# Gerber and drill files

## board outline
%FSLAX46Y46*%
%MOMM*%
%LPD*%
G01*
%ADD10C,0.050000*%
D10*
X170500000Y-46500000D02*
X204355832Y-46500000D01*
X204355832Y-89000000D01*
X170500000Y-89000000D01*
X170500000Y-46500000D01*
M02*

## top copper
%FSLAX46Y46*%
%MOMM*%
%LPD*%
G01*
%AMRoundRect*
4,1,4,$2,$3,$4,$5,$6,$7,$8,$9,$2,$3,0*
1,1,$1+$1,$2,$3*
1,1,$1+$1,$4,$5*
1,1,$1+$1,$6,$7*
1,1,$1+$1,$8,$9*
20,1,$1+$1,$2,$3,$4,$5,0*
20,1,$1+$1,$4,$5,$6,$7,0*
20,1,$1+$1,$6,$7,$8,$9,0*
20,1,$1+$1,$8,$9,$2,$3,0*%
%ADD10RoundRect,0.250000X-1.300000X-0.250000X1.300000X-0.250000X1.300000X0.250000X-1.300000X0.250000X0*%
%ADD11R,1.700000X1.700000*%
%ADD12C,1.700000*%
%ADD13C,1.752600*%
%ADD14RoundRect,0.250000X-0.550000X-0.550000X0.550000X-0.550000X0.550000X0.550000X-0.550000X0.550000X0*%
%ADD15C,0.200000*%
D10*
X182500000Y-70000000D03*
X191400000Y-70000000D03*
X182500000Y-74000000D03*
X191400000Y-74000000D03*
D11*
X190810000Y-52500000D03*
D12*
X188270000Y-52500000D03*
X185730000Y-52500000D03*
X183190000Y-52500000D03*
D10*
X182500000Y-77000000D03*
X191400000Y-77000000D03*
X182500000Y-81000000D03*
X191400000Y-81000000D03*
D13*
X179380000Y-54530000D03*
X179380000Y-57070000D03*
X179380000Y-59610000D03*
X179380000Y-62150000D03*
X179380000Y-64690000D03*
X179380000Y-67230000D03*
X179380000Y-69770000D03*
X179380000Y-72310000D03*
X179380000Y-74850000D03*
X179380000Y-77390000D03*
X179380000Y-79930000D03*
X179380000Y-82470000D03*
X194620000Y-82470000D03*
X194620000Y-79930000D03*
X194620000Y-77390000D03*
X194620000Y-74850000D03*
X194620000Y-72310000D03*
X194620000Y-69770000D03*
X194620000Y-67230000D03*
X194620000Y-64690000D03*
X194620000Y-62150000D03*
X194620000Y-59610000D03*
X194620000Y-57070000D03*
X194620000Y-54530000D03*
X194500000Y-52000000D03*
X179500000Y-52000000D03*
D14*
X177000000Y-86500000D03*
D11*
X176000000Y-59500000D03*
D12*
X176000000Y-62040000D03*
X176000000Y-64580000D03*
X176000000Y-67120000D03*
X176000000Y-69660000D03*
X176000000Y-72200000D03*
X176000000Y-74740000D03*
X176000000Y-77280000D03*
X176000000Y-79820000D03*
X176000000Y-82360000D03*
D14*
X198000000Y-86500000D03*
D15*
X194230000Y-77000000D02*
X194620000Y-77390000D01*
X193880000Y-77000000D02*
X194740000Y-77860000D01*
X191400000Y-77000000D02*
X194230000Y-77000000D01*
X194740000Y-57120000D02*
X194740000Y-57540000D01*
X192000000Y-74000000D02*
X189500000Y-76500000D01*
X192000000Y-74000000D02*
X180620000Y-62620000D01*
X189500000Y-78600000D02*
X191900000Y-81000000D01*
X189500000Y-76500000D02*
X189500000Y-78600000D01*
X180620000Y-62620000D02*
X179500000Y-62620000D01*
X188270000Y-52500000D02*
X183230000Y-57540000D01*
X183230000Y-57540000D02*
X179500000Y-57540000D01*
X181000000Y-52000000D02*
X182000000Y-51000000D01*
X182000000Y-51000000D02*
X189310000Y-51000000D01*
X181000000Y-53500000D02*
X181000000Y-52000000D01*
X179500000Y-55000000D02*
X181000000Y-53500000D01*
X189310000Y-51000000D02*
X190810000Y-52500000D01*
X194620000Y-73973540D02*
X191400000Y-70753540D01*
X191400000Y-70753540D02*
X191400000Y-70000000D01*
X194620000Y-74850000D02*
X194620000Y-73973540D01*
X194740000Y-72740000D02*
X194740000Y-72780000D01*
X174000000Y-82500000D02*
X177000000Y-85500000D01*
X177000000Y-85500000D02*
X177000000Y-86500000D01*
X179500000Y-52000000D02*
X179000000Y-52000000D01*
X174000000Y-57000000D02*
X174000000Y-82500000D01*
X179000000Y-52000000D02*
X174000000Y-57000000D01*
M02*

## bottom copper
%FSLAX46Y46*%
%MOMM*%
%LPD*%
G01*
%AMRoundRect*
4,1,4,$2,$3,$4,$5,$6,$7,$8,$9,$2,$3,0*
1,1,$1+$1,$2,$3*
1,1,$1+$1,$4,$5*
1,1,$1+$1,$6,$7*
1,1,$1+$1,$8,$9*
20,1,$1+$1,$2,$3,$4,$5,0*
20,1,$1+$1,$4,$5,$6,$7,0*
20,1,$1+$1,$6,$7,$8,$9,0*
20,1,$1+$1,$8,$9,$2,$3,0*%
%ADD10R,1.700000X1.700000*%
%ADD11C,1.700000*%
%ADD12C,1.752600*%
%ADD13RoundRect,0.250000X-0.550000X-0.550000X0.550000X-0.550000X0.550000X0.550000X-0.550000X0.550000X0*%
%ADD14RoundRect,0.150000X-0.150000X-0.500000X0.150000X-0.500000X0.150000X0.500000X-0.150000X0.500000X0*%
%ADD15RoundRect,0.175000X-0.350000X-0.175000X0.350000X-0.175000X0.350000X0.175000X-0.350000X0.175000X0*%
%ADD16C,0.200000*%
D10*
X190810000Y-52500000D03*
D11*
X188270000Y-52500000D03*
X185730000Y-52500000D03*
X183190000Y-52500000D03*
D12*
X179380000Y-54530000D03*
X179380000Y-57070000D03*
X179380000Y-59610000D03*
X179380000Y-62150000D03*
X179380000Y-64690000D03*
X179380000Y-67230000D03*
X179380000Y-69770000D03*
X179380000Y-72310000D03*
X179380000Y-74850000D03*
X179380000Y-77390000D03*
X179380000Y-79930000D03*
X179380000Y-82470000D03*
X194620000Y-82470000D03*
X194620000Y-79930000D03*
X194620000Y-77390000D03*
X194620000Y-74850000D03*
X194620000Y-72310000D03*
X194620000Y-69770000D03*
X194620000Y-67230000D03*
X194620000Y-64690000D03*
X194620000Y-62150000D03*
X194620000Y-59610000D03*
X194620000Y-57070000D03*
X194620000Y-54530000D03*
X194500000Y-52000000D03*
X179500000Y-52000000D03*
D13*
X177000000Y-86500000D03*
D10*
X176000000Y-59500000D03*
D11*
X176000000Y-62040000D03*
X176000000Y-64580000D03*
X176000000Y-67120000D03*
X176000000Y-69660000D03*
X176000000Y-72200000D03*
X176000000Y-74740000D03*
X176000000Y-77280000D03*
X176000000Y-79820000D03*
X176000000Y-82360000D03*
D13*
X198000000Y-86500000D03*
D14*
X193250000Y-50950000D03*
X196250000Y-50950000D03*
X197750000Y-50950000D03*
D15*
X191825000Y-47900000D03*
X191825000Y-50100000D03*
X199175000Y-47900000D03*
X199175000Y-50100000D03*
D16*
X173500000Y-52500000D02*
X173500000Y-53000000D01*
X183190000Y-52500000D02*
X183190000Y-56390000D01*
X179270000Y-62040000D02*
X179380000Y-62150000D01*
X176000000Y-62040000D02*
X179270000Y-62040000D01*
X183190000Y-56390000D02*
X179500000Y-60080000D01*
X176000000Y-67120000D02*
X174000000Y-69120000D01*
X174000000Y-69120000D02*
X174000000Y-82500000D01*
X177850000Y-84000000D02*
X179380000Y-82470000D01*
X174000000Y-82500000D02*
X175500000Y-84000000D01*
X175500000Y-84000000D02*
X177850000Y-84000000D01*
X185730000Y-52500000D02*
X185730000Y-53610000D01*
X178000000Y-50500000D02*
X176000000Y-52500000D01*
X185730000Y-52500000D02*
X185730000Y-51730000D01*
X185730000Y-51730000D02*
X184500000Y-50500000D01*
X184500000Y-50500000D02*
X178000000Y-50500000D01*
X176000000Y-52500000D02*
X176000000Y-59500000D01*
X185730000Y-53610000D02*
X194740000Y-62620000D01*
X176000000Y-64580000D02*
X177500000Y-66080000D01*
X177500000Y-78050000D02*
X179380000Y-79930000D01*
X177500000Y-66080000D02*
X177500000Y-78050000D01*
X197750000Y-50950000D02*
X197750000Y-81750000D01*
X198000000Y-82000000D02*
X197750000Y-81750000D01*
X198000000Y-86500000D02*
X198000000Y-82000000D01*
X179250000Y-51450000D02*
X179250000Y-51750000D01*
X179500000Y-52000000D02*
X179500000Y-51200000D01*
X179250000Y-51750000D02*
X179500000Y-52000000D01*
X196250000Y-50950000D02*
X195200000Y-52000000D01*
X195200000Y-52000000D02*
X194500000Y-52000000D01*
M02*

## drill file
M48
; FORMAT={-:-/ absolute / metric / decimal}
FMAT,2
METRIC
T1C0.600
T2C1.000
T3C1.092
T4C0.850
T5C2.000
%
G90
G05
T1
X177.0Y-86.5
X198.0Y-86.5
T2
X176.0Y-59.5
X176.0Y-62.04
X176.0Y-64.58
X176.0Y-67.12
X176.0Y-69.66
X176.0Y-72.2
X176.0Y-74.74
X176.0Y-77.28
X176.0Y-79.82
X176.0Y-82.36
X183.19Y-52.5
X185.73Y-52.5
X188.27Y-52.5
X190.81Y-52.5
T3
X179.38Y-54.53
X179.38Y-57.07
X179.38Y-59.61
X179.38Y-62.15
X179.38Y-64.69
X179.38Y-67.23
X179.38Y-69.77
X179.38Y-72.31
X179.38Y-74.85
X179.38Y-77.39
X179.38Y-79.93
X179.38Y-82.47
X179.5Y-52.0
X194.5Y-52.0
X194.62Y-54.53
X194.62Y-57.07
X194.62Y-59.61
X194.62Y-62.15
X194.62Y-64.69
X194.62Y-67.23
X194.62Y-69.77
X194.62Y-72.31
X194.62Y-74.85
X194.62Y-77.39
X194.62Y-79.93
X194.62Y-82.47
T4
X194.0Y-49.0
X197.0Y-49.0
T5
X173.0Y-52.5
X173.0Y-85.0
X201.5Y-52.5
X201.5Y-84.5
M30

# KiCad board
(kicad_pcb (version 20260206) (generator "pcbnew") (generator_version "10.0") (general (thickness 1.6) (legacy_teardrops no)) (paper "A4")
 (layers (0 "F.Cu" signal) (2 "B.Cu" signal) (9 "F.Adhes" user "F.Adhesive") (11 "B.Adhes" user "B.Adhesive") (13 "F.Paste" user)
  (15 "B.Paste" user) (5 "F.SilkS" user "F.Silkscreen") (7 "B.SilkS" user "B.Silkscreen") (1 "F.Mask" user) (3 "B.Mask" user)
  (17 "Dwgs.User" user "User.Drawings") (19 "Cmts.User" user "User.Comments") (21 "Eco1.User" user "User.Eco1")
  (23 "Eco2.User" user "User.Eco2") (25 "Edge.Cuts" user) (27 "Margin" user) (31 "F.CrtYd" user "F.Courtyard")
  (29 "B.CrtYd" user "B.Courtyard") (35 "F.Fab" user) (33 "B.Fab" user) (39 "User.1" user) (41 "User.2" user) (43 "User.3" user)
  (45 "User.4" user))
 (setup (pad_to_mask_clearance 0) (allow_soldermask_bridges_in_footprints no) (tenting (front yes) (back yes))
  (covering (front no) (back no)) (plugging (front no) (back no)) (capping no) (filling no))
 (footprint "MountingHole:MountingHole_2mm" (layer "F.Cu") (at 201.5 52.5)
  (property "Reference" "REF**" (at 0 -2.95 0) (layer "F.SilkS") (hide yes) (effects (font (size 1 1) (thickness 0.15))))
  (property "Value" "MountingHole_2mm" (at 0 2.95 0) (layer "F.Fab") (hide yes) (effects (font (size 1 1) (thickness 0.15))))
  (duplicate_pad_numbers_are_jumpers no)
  (pad "" np_thru_hole circle (at 0 0) (size 2 2) (drill 2) (layers "*.Cu" "*.Mask")))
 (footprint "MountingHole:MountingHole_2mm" (layer "F.Cu") (at 201.5 84.5)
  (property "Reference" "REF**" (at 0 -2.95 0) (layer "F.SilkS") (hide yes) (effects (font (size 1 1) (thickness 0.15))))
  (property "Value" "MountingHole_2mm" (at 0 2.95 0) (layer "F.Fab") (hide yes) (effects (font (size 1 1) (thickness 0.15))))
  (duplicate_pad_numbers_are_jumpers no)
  (pad "" np_thru_hole circle (at 0 0) (size 2 2) (drill 2) (layers "*.Cu" "*.Mask")))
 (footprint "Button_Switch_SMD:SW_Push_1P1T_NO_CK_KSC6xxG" (layer "F.Cu") (at 186.95 72)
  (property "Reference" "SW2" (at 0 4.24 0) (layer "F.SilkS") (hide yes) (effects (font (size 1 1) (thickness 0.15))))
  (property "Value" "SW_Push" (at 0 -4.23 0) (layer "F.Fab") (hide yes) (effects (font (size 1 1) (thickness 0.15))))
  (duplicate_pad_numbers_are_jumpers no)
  (pad "1" smd roundrect (at -4.45 -2) (size 3.1 1) (layers "F.Cu" "F.Mask" "F.Paste") (roundrect_rratio 0.25) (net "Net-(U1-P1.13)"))
  (pad "1" smd roundrect (at 4.45 -2) (size 3.1 1) (layers "F.Cu" "F.Mask" "F.Paste") (roundrect_rratio 0.25) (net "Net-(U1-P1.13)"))
  (pad "2" smd roundrect (at -4.45 2) (size 3.1 1) (layers "F.Cu" "F.Mask" "F.Paste") (roundrect_rratio 0.25) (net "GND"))
  (pad "2" smd roundrect (at 4.45 2) (size 3.1 1) (layers "F.Cu" "F.Mask" "F.Paste") (roundrect_rratio 0.25) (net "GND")))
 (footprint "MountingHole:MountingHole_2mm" (layer "F.Cu") (at 173 52.5)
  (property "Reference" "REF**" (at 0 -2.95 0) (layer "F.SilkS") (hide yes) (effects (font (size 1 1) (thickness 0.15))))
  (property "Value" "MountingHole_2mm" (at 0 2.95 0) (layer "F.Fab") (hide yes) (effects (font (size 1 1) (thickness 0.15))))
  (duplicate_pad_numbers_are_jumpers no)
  (pad "" np_thru_hole circle (at 0 0) (size 2 2) (drill 2) (layers "*.Cu" "*.Mask")))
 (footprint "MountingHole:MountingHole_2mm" (layer "F.Cu") (at 173 85)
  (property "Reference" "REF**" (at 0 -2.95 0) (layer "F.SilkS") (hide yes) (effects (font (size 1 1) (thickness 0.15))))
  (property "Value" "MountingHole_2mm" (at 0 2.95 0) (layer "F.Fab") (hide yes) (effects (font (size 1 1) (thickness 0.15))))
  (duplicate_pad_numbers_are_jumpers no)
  (pad "" np_thru_hole circle (at 0 0) (size 2 2) (drill 2) (layers "*.Cu" "*.Mask")))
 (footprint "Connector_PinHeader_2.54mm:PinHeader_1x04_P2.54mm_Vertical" (layer "F.Cu") (at 190.81 52.5 -90)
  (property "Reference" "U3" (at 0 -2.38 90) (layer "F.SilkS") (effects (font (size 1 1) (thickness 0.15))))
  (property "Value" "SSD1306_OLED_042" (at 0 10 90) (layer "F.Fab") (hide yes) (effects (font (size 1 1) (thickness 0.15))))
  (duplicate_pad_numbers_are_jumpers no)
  (pad "1" thru_hole rect (at 0 0 270) (size 1.7 1.7) (drill 1) (layers "*.Cu" "*.Mask") (remove_unused_layers no)
   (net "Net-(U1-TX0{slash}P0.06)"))
  (pad "2" thru_hole circle (at 0 2.54 270) (size 1.7 1.7) (drill 1) (layers "*.Cu" "*.Mask") (remove_unused_layers no)
   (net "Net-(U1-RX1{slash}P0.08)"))
  (pad "3" thru_hole circle (at 0 5.08 270) (size 1.7 1.7) (drill 1) (layers "*.Cu" "*.Mask") (remove_unused_layers no) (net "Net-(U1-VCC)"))
  (pad "4" thru_hole circle (at 0 7.62 270) (size 1.7 1.7) (drill 1) (layers "*.Cu" "*.Mask") (remove_unused_layers no) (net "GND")))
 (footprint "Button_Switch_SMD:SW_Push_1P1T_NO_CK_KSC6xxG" (layer "F.Cu") (at 186.95 79)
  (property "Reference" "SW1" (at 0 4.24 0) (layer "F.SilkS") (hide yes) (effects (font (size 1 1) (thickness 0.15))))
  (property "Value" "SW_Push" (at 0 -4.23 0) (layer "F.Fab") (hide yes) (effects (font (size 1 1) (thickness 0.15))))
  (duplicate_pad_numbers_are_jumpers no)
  (pad "1" smd roundrect (at -4.45 -2) (size 3.1 1) (layers "F.Cu" "F.Mask" "F.Paste") (roundrect_rratio 0.25) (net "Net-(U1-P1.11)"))
  (pad "1" smd roundrect (at 4.45 -2) (size 3.1 1) (layers "F.Cu" "F.Mask" "F.Paste") (roundrect_rratio 0.25) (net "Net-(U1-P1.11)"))
  (pad "2" smd roundrect (at -4.45 2) (size 3.1 1) (layers "F.Cu" "F.Mask" "F.Paste") (roundrect_rratio 0.25) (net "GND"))
  (pad "2" smd roundrect (at 4.45 2) (size 3.1 1) (layers "F.Cu" "F.Mask" "F.Paste") (roundrect_rratio 0.25) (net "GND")))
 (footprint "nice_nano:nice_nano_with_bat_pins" (layer "F.Cu") (at 187 68.5 -90)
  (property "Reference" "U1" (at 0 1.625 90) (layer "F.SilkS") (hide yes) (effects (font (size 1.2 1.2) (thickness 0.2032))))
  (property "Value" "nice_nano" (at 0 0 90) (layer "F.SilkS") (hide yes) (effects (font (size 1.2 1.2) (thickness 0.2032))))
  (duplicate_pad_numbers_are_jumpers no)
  (pad "1" thru_hole circle (at -13.97 7.62 270) (size 1.7526 1.7526) (drill 1.0922) (layers "*.Cu" "*.SilkS" "*.Mask")
   (remove_unused_layers no) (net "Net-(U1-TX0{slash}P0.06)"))
  (pad "2" thru_hole circle (at -11.43 7.62 270) (size 1.7526 1.7526) (drill 1.0922) (layers "*.Cu" "*.SilkS" "*.Mask")
   (remove_unused_layers no) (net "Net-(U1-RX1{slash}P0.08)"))
  (pad "3" thru_hole circle (at -8.89 7.62 270) (size 1.7526 1.7526) (drill 1.0922) (layers "*.Cu" "*.SilkS" "*.Mask")
   (remove_unused_layers no) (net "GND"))
  (pad "4" thru_hole circle (at -6.35 7.62 270) (size 1.7526 1.7526) (drill 1.0922) (layers "*.Cu" "*.SilkS" "*.Mask")
   (remove_unused_layers no) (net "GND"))
  (pad "5" thru_hole circle (at -3.81 7.62 270) (size 1.7526 1.7526) (drill 1.0922) (layers "*.Cu" "*.SilkS" "*.Mask")
   (remove_unused_layers no) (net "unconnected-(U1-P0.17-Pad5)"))
  (pad "6" thru_hole circle (at -1.27 7.62 270) (size 1.7526 1.7526) (drill 1.0922) (layers "*.Cu" "*.SilkS" "*.Mask")
   (remove_unused_layers no) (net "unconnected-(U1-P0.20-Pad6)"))
  (pad "7" thru_hole circle (at 1.27 7.62 270) (size 1.7526 1.7526) (drill 1.0922) (layers "*.Cu" "*.SilkS" "*.Mask")
   (remove_unused_layers no) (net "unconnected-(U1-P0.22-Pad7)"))
  (pad "8" thru_hole circle (at 3.81 7.62 270) (size 1.7526 1.7526) (drill 1.0922) (layers "*.Cu" "*.SilkS" "*.Mask")
   (remove_unused_layers no) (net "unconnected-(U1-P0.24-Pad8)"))
  (pad "9" thru_hole circle (at 6.35 7.62 270) (size 1.7526 1.7526) (drill 1.0922) (layers "*.Cu" "*.SilkS" "*.Mask")
   (remove_unused_layers no) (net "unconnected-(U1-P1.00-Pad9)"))
  (pad "10" thru_hole circle (at 8.89 7.62 270) (size 1.7526 1.7526) (drill 1.0922) (layers "*.Cu" "*.SilkS" "*.Mask")
   (remove_unused_layers no) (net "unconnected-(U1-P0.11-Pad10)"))
  (pad "11" thru_hole circle (at 11.43 7.62 270) (size 1.7526 1.7526) (drill 1.0922) (layers "*.Cu" "*.SilkS" "*.Mask")
   (remove_unused_layers no) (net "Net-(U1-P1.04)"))
  (pad "12" thru_hole circle (at 13.97 7.62 270) (size 1.7526 1.7526) (drill 1.0922) (layers "*.Cu" "*.SilkS" "*.Mask")
   (remove_unused_layers no) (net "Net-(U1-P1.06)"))
  (pad "13" thru_hole circle (at 13.97 -7.62 270) (size 1.7526 1.7526) (drill 1.0922) (layers "*.Cu" "*.SilkS" "*.Mask")
   (remove_unused_layers no) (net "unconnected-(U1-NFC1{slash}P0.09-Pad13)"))
  (pad "14" thru_hole circle (at 11.43 -7.62 270) (size 1.7526 1.7526) (drill 1.0922) (layers "*.Cu" "*.SilkS" "*.Mask")
   (remove_unused_layers no) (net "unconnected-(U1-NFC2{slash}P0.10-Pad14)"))
  (pad "15" thru_hole circle (at 8.89 -7.62 270) (size 1.7526 1.7526) (drill 1.0922) (layers "*.Cu" "*.SilkS" "*.Mask")
   (remove_unused_layers no) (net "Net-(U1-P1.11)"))
  (pad "16" thru_hole circle (at 6.35 -7.62 270) (size 1.7526 1.7526) (drill 1.0922) (layers "*.Cu" "*.SilkS" "*.Mask")
   (remove_unused_layers no) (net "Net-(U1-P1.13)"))
  (pad "17" thru_hole circle (at 3.81 -7.62 270) (size 1.7526 1.7526) (drill 1.0922) (layers "*.Cu" "*.SilkS" "*.Mask")
   (remove_unused_layers no) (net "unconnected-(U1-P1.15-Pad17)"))
  (pad "18" thru_hole circle (at 1.27 -7.62 270) (size 1.7526 1.7526) (drill 1.0922) (layers "*.Cu" "*.SilkS" "*.Mask")
   (remove_unused_layers no) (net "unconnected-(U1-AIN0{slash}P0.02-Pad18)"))
  (pad "19" thru_hole circle (at -1.27 -7.62 270) (size 1.7526 1.7526) (drill 1.0922) (layers "*.Cu" "*.SilkS" "*.Mask")
   (remove_unused_layers no) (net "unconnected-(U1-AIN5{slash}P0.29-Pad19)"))
  (pad "20" thru_hole circle (at -3.81 -7.62 270) (size 1.7526 1.7526) (drill 1.0922) (layers "*.Cu" "*.SilkS" "*.Mask")
   (remove_unused_layers no) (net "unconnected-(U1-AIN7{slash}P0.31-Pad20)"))
  (pad "21" thru_hole circle (at -6.35 -7.62 270) (size 1.7526 1.7526) (drill 1.0922) (layers "*.Cu" "*.SilkS" "*.Mask")
   (remove_unused_layers no) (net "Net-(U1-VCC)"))
  (pad "22" thru_hole circle (at -8.89 -7.62 270) (size 1.7526 1.7526) (drill 1.0922) (layers "*.Cu" "*.SilkS" "*.Mask")
   (remove_unused_layers no) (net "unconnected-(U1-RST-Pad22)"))
  (pad "23" thru_hole circle (at -11.43 -7.62 270) (size 1.7526 1.7526) (drill 1.0922) (layers "*.Cu" "*.SilkS" "*.Mask")
   (remove_unused_layers no) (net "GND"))
  (pad "24" thru_hole circle (at -13.97 -7.62 270) (size 1.7526 1.7526) (drill 1.0922) (layers "*.Cu" "*.SilkS" "*.Mask")
   (remove_unused_layers no) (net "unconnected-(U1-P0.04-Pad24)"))
  (pad "25" thru_hole circle (at -16.5 -7.5 270) (size 1.7526 1.7526) (drill 1.0922) (layers "*.Cu" "*.SilkS" "*.Mask")
   (remove_unused_layers no) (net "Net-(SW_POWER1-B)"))
  (pad "26" thru_hole circle (at -16.5 7.5 270) (size 1.7526 1.7526) (drill 1.0922) (layers "*.Cu" "*.SilkS" "*.Mask")
   (remove_unused_layers no) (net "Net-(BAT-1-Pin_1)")))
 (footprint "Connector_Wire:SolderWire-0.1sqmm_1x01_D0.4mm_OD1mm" (layer "B.Cu") (at 177 86.5)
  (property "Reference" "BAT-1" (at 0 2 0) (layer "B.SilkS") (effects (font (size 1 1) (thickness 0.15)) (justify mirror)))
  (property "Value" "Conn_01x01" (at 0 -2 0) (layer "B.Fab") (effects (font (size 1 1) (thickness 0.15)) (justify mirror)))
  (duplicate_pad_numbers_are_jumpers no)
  (pad "1" thru_hole roundrect (at 0 0) (size 1.6 1.6) (drill 0.6) (layers "*.Cu" "*.Mask") (remove_unused_layers no)
   (roundrect_rratio 0.15625) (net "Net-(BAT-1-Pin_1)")))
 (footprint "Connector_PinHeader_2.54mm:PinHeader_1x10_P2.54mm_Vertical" (layer "B.Cu") (at 176 59.5 180)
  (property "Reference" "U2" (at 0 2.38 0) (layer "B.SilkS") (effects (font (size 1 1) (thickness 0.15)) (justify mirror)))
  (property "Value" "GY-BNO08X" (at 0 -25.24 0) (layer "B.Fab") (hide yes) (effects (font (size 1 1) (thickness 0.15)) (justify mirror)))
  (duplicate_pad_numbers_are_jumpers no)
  (pad "1" thru_hole rect (at 0 0 180) (size 1.7 1.7) (drill 1) (layers "*.Cu" "*.Mask") (remove_unused_layers no) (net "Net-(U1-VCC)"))
  (pad "2" thru_hole circle (at 0 -2.54 180) (size 1.7 1.7) (drill 1) (layers "*.Cu" "*.Mask") (remove_unused_layers no) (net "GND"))
  (pad "3" thru_hole circle (at 0 -5.08 180) (size 1.7 1.7) (drill 1) (layers "*.Cu" "*.Mask") (remove_unused_layers no)
   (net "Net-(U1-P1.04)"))
  (pad "4" thru_hole circle (at 0 -7.62 180) (size 1.7 1.7) (drill 1) (layers "*.Cu" "*.Mask") (remove_unused_layers no)
   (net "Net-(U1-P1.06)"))
  (pad "5" thru_hole circle (at 0 -10.16 180) (size 1.7 1.7) (drill 1) (layers "*.Cu" "*.Mask") (remove_unused_layers no)
   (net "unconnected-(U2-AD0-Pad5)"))
  (pad "6" thru_hole circle (at 0 -12.7 180) (size 1.7 1.7) (drill 1) (layers "*.Cu" "*.Mask") (remove_unused_layers no)
   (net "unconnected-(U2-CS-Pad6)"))
  (pad "7" thru_hole circle (at 0 -15.24 180) (size 1.7 1.7) (drill 1) (layers "*.Cu" "*.Mask") (remove_unused_layers no)
   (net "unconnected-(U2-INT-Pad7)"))
  (pad "8" thru_hole circle (at 0 -17.78 180) (size 1.7 1.7) (drill 1) (layers "*.Cu" "*.Mask") (remove_unused_layers no)
   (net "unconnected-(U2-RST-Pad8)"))
  (pad "9" thru_hole circle (at 0 -20.32 180) (size 1.7 1.7) (drill 1) (layers "*.Cu" "*.Mask") (remove_unused_layers no)
   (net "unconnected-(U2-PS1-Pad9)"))
  (pad "10" thru_hole circle (at 0 -22.86 180) (size 1.7 1.7) (drill 1) (layers "*.Cu" "*.Mask") (remove_unused_layers no)
   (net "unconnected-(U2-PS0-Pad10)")))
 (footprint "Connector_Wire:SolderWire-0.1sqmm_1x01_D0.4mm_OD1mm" (layer "B.Cu") (at 198 86.5)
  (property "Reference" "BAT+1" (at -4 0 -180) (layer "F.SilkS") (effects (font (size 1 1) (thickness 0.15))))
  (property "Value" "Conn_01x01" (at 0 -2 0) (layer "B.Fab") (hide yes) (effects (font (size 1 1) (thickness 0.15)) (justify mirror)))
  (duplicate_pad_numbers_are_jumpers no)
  (pad "1" thru_hole roundrect (at 0 0) (size 1.6 1.6) (drill 0.6) (layers "*.Cu" "*.Mask") (remove_unused_layers no)
   (roundrect_rratio 0.15625) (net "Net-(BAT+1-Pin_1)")))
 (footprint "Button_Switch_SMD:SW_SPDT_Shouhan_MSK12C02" (layer "B.Cu") (at 195.5 49)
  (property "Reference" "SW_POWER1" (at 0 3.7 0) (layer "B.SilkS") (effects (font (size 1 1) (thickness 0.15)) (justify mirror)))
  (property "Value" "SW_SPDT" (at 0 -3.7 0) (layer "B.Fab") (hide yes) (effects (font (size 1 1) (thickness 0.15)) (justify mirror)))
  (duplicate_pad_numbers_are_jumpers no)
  (pad "" np_thru_hole circle (at -1.5 0) (size 0.85 0.85) (drill 0.85) (layers "*.Mask"))
  (pad "" np_thru_hole circle (at 1.5 0) (size 0.85 0.85) (drill 0.85) (layers "*.Mask"))
  (pad "1" smd roundrect (at -2.25 1.95) (size 0.6 1.3) (layers "B.Cu" "B.Mask" "B.Paste") (roundrect_rratio 0.25)
   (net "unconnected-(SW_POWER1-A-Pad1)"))
  (pad "2" smd roundrect (at 0.75 1.95) (size 0.6 1.3) (layers "B.Cu" "B.Mask" "B.Paste") (roundrect_rratio 0.25) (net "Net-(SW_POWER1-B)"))
  (pad "3" smd roundrect (at 2.25 1.95) (size 0.6 1.3) (layers "B.Cu" "B.Mask" "B.Paste") (roundrect_rratio 0.25) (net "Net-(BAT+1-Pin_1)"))
  (pad "SH" smd roundrect (at -3.675 -1.1) (size 1.05 0.7) (layers "B.Cu" "B.Mask" "B.Paste") (roundrect_rratio 0.25))
  (pad "SH" smd roundrect (at -3.675 1.1) (size 1.05 0.7) (layers "B.Cu" "B.Mask" "B.Paste") (roundrect_rratio 0.25))
  (pad "SH" smd roundrect (at 3.675 -1.1) (size 1.05 0.7) (layers "B.Cu" "B.Mask" "B.Paste") (roundrect_rratio 0.25))
  (pad "SH" smd roundrect (at 3.675 1.1) (size 1.05 0.7) (layers "B.Cu" "B.Mask" "B.Paste") (roundrect_rratio 0.25)))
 (gr_rect (start 170.5 46.5) (end 204.355832 89) (stroke (width 0.05) (type default)) (fill no) (layer "Edge.Cuts"))
 (segment (start 173.5 52.5) (end 173.5 53) (width 0.2) (layer "B.Cu") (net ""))
 (segment (start 194.23 77) (end 194.62 77.39) (width 0.2) (layer "F.Cu") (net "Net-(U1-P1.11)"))
 (segment (start 193.88 77) (end 194.74 77.86) (width 0.2) (layer "F.Cu") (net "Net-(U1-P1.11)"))
 (segment (start 191.4 77) (end 194.23 77) (width 0.2) (layer "F.Cu") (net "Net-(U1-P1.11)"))
 (segment (start 194.74 57.12) (end 194.74 57.54) (width 0.2) (layer "F.Cu") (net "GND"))
 (segment (start 192 74) (end 189.5 76.5) (width 0.2) (layer "F.Cu") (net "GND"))
 (segment (start 192 74) (end 180.62 62.62) (width 0.2) (layer "F.Cu") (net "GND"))
 (segment (start 189.5 78.6) (end 191.9 81) (width 0.2) (layer "F.Cu") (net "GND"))
 (segment (start 189.5 76.5) (end 189.5 78.6) (width 0.2) (layer "F.Cu") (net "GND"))
 (segment (start 180.62 62.62) (end 179.5 62.62) (width 0.2) (layer "F.Cu") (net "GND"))
 (segment (start 183.19 52.5) (end 183.19 56.39) (width 0.2) (layer "B.Cu") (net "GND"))
 (segment (start 179.27 62.04) (end 179.38 62.15) (width 0.2) (layer "B.Cu") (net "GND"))
 (segment (start 176 62.04) (end 179.27 62.04) (width 0.2) (layer "B.Cu") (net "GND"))
 (segment (start 183.19 56.39) (end 179.5 60.08) (width 0.2) (layer "B.Cu") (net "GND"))
 (segment (start 176 67.12) (end 174 69.12) (width 0.2) (layer "B.Cu") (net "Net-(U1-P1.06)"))
 (segment (start 174 69.12) (end 174 82.5) (width 0.2) (layer "B.Cu") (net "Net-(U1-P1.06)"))
 (segment (start 177.85 84) (end 179.38 82.47) (width 0.2) (layer "B.Cu") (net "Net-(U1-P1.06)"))
 (segment (start 174 82.5) (end 175.5 84) (width 0.2) (layer "B.Cu") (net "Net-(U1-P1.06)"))
 (segment (start 175.5 84) (end 177.85 84) (width 0.2) (layer "B.Cu") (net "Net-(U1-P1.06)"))
 (segment (start 188.27 52.5) (end 183.23 57.54) (width 0.2) (layer "F.Cu") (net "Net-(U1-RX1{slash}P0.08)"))
 (segment (start 183.23 57.54) (end 179.5 57.54) (width 0.2) (layer "F.Cu") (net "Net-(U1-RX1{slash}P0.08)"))
 (segment (start 185.73 52.5) (end 185.73 53.61) (width 0.2) (layer "B.Cu") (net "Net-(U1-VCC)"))
 (segment (start 178 50.5) (end 176 52.5) (width 0.2) (layer "B.Cu") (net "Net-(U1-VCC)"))
 (segment (start 185.73 52.5) (end 185.73 51.73) (width 0.2) (layer "B.Cu") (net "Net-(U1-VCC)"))
 (segment (start 185.73 51.73) (end 184.5 50.5) (width 0.2) (layer "B.Cu") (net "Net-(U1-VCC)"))
 (segment (start 184.5 50.5) (end 178 50.5) (width 0.2) (layer "B.Cu") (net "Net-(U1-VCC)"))
 (segment (start 176 52.5) (end 176 59.5) (width 0.2) (layer "B.Cu") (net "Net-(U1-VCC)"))
 (segment (start 185.73 53.61) (end 194.74 62.62) (width 0.2) (layer "B.Cu") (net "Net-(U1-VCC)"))
 (segment (start 181 52) (end 182 51) (width 0.2) (layer "F.Cu") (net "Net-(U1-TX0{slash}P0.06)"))
 (segment (start 182 51) (end 189.31 51) (width 0.2) (layer "F.Cu") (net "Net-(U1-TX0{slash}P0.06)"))
 (segment (start 181 53.5) (end 181 52) (width 0.2) (layer "F.Cu") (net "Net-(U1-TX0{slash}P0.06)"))
 (segment (start 179.5 55) (end 181 53.5) (width 0.2) (layer "F.Cu") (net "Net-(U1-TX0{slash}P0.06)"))
 (segment (start 189.31 51) (end 190.81 52.5) (width 0.2) (layer "F.Cu") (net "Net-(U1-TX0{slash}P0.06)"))
 (segment (start 176 64.58) (end 177.5 66.08) (width 0.2) (layer "B.Cu") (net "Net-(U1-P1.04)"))
 (segment (start 177.5 78.05) (end 179.38 79.93) (width 0.2) (layer "B.Cu") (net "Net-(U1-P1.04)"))
 (segment (start 177.5 66.08) (end 177.5 78.05) (width 0.2) (layer "B.Cu") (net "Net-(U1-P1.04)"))
 (segment (start 194.62 73.97354) (end 191.4 70.75354) (width 0.2) (layer "F.Cu") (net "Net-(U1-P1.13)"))
 (segment (start 191.4 70.75354) (end 191.4 70) (width 0.2) (layer "F.Cu") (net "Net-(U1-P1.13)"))
 (segment (start 194.62 74.85) (end 194.62 73.97354) (width 0.2) (layer "F.Cu") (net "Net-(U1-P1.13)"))
 (segment (start 194.74 72.74) (end 194.74 72.78) (width 0.2) (layer "F.Cu") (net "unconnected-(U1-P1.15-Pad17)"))
 (segment (start 197.75 50.95) (end 197.75 81.75) (width 0.2) (layer "B.Cu") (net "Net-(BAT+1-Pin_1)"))
 (segment (start 198 82) (end 197.75 81.75) (width 0.2) (layer "B.Cu") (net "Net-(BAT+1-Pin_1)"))
 (segment (start 198 86.5) (end 198 82) (width 0.2) (layer "B.Cu") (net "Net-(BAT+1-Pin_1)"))
 (segment (start 174 82.5) (end 177 85.5) (width 0.2) (layer "F.Cu") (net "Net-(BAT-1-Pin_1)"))
 (segment (start 177 85.5) (end 177 86.5) (width 0.2) (layer "F.Cu") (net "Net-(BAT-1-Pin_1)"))
 (segment (start 179.5 52) (end 179 52) (width 0.2) (layer "F.Cu") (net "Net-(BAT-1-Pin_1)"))
 (segment (start 174 57) (end 174 82.5) (width 0.2) (layer "F.Cu") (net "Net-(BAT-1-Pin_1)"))
 (segment (start 179 52) (end 174 57) (width 0.2) (layer "F.Cu") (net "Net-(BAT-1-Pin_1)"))
 (segment (start 179.25 51.45) (end 179.25 51.75) (width 0.2) (layer "B.Cu") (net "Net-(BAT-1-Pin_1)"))
 (segment (start 179.5 52) (end 179.5 51.2) (width 0.2) (layer "B.Cu") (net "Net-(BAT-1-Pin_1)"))
 (segment (start 179.25 51.75) (end 179.5 52) (width 0.2) (layer "B.Cu") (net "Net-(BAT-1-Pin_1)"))
 (segment (start 196.25 50.95) (end 195.2 52) (width 0.2) (layer "B.Cu") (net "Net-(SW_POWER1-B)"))
 (segment (start 195.2 52) (end 194.5 52) (width 0.2) (layer "B.Cu") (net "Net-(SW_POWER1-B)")))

